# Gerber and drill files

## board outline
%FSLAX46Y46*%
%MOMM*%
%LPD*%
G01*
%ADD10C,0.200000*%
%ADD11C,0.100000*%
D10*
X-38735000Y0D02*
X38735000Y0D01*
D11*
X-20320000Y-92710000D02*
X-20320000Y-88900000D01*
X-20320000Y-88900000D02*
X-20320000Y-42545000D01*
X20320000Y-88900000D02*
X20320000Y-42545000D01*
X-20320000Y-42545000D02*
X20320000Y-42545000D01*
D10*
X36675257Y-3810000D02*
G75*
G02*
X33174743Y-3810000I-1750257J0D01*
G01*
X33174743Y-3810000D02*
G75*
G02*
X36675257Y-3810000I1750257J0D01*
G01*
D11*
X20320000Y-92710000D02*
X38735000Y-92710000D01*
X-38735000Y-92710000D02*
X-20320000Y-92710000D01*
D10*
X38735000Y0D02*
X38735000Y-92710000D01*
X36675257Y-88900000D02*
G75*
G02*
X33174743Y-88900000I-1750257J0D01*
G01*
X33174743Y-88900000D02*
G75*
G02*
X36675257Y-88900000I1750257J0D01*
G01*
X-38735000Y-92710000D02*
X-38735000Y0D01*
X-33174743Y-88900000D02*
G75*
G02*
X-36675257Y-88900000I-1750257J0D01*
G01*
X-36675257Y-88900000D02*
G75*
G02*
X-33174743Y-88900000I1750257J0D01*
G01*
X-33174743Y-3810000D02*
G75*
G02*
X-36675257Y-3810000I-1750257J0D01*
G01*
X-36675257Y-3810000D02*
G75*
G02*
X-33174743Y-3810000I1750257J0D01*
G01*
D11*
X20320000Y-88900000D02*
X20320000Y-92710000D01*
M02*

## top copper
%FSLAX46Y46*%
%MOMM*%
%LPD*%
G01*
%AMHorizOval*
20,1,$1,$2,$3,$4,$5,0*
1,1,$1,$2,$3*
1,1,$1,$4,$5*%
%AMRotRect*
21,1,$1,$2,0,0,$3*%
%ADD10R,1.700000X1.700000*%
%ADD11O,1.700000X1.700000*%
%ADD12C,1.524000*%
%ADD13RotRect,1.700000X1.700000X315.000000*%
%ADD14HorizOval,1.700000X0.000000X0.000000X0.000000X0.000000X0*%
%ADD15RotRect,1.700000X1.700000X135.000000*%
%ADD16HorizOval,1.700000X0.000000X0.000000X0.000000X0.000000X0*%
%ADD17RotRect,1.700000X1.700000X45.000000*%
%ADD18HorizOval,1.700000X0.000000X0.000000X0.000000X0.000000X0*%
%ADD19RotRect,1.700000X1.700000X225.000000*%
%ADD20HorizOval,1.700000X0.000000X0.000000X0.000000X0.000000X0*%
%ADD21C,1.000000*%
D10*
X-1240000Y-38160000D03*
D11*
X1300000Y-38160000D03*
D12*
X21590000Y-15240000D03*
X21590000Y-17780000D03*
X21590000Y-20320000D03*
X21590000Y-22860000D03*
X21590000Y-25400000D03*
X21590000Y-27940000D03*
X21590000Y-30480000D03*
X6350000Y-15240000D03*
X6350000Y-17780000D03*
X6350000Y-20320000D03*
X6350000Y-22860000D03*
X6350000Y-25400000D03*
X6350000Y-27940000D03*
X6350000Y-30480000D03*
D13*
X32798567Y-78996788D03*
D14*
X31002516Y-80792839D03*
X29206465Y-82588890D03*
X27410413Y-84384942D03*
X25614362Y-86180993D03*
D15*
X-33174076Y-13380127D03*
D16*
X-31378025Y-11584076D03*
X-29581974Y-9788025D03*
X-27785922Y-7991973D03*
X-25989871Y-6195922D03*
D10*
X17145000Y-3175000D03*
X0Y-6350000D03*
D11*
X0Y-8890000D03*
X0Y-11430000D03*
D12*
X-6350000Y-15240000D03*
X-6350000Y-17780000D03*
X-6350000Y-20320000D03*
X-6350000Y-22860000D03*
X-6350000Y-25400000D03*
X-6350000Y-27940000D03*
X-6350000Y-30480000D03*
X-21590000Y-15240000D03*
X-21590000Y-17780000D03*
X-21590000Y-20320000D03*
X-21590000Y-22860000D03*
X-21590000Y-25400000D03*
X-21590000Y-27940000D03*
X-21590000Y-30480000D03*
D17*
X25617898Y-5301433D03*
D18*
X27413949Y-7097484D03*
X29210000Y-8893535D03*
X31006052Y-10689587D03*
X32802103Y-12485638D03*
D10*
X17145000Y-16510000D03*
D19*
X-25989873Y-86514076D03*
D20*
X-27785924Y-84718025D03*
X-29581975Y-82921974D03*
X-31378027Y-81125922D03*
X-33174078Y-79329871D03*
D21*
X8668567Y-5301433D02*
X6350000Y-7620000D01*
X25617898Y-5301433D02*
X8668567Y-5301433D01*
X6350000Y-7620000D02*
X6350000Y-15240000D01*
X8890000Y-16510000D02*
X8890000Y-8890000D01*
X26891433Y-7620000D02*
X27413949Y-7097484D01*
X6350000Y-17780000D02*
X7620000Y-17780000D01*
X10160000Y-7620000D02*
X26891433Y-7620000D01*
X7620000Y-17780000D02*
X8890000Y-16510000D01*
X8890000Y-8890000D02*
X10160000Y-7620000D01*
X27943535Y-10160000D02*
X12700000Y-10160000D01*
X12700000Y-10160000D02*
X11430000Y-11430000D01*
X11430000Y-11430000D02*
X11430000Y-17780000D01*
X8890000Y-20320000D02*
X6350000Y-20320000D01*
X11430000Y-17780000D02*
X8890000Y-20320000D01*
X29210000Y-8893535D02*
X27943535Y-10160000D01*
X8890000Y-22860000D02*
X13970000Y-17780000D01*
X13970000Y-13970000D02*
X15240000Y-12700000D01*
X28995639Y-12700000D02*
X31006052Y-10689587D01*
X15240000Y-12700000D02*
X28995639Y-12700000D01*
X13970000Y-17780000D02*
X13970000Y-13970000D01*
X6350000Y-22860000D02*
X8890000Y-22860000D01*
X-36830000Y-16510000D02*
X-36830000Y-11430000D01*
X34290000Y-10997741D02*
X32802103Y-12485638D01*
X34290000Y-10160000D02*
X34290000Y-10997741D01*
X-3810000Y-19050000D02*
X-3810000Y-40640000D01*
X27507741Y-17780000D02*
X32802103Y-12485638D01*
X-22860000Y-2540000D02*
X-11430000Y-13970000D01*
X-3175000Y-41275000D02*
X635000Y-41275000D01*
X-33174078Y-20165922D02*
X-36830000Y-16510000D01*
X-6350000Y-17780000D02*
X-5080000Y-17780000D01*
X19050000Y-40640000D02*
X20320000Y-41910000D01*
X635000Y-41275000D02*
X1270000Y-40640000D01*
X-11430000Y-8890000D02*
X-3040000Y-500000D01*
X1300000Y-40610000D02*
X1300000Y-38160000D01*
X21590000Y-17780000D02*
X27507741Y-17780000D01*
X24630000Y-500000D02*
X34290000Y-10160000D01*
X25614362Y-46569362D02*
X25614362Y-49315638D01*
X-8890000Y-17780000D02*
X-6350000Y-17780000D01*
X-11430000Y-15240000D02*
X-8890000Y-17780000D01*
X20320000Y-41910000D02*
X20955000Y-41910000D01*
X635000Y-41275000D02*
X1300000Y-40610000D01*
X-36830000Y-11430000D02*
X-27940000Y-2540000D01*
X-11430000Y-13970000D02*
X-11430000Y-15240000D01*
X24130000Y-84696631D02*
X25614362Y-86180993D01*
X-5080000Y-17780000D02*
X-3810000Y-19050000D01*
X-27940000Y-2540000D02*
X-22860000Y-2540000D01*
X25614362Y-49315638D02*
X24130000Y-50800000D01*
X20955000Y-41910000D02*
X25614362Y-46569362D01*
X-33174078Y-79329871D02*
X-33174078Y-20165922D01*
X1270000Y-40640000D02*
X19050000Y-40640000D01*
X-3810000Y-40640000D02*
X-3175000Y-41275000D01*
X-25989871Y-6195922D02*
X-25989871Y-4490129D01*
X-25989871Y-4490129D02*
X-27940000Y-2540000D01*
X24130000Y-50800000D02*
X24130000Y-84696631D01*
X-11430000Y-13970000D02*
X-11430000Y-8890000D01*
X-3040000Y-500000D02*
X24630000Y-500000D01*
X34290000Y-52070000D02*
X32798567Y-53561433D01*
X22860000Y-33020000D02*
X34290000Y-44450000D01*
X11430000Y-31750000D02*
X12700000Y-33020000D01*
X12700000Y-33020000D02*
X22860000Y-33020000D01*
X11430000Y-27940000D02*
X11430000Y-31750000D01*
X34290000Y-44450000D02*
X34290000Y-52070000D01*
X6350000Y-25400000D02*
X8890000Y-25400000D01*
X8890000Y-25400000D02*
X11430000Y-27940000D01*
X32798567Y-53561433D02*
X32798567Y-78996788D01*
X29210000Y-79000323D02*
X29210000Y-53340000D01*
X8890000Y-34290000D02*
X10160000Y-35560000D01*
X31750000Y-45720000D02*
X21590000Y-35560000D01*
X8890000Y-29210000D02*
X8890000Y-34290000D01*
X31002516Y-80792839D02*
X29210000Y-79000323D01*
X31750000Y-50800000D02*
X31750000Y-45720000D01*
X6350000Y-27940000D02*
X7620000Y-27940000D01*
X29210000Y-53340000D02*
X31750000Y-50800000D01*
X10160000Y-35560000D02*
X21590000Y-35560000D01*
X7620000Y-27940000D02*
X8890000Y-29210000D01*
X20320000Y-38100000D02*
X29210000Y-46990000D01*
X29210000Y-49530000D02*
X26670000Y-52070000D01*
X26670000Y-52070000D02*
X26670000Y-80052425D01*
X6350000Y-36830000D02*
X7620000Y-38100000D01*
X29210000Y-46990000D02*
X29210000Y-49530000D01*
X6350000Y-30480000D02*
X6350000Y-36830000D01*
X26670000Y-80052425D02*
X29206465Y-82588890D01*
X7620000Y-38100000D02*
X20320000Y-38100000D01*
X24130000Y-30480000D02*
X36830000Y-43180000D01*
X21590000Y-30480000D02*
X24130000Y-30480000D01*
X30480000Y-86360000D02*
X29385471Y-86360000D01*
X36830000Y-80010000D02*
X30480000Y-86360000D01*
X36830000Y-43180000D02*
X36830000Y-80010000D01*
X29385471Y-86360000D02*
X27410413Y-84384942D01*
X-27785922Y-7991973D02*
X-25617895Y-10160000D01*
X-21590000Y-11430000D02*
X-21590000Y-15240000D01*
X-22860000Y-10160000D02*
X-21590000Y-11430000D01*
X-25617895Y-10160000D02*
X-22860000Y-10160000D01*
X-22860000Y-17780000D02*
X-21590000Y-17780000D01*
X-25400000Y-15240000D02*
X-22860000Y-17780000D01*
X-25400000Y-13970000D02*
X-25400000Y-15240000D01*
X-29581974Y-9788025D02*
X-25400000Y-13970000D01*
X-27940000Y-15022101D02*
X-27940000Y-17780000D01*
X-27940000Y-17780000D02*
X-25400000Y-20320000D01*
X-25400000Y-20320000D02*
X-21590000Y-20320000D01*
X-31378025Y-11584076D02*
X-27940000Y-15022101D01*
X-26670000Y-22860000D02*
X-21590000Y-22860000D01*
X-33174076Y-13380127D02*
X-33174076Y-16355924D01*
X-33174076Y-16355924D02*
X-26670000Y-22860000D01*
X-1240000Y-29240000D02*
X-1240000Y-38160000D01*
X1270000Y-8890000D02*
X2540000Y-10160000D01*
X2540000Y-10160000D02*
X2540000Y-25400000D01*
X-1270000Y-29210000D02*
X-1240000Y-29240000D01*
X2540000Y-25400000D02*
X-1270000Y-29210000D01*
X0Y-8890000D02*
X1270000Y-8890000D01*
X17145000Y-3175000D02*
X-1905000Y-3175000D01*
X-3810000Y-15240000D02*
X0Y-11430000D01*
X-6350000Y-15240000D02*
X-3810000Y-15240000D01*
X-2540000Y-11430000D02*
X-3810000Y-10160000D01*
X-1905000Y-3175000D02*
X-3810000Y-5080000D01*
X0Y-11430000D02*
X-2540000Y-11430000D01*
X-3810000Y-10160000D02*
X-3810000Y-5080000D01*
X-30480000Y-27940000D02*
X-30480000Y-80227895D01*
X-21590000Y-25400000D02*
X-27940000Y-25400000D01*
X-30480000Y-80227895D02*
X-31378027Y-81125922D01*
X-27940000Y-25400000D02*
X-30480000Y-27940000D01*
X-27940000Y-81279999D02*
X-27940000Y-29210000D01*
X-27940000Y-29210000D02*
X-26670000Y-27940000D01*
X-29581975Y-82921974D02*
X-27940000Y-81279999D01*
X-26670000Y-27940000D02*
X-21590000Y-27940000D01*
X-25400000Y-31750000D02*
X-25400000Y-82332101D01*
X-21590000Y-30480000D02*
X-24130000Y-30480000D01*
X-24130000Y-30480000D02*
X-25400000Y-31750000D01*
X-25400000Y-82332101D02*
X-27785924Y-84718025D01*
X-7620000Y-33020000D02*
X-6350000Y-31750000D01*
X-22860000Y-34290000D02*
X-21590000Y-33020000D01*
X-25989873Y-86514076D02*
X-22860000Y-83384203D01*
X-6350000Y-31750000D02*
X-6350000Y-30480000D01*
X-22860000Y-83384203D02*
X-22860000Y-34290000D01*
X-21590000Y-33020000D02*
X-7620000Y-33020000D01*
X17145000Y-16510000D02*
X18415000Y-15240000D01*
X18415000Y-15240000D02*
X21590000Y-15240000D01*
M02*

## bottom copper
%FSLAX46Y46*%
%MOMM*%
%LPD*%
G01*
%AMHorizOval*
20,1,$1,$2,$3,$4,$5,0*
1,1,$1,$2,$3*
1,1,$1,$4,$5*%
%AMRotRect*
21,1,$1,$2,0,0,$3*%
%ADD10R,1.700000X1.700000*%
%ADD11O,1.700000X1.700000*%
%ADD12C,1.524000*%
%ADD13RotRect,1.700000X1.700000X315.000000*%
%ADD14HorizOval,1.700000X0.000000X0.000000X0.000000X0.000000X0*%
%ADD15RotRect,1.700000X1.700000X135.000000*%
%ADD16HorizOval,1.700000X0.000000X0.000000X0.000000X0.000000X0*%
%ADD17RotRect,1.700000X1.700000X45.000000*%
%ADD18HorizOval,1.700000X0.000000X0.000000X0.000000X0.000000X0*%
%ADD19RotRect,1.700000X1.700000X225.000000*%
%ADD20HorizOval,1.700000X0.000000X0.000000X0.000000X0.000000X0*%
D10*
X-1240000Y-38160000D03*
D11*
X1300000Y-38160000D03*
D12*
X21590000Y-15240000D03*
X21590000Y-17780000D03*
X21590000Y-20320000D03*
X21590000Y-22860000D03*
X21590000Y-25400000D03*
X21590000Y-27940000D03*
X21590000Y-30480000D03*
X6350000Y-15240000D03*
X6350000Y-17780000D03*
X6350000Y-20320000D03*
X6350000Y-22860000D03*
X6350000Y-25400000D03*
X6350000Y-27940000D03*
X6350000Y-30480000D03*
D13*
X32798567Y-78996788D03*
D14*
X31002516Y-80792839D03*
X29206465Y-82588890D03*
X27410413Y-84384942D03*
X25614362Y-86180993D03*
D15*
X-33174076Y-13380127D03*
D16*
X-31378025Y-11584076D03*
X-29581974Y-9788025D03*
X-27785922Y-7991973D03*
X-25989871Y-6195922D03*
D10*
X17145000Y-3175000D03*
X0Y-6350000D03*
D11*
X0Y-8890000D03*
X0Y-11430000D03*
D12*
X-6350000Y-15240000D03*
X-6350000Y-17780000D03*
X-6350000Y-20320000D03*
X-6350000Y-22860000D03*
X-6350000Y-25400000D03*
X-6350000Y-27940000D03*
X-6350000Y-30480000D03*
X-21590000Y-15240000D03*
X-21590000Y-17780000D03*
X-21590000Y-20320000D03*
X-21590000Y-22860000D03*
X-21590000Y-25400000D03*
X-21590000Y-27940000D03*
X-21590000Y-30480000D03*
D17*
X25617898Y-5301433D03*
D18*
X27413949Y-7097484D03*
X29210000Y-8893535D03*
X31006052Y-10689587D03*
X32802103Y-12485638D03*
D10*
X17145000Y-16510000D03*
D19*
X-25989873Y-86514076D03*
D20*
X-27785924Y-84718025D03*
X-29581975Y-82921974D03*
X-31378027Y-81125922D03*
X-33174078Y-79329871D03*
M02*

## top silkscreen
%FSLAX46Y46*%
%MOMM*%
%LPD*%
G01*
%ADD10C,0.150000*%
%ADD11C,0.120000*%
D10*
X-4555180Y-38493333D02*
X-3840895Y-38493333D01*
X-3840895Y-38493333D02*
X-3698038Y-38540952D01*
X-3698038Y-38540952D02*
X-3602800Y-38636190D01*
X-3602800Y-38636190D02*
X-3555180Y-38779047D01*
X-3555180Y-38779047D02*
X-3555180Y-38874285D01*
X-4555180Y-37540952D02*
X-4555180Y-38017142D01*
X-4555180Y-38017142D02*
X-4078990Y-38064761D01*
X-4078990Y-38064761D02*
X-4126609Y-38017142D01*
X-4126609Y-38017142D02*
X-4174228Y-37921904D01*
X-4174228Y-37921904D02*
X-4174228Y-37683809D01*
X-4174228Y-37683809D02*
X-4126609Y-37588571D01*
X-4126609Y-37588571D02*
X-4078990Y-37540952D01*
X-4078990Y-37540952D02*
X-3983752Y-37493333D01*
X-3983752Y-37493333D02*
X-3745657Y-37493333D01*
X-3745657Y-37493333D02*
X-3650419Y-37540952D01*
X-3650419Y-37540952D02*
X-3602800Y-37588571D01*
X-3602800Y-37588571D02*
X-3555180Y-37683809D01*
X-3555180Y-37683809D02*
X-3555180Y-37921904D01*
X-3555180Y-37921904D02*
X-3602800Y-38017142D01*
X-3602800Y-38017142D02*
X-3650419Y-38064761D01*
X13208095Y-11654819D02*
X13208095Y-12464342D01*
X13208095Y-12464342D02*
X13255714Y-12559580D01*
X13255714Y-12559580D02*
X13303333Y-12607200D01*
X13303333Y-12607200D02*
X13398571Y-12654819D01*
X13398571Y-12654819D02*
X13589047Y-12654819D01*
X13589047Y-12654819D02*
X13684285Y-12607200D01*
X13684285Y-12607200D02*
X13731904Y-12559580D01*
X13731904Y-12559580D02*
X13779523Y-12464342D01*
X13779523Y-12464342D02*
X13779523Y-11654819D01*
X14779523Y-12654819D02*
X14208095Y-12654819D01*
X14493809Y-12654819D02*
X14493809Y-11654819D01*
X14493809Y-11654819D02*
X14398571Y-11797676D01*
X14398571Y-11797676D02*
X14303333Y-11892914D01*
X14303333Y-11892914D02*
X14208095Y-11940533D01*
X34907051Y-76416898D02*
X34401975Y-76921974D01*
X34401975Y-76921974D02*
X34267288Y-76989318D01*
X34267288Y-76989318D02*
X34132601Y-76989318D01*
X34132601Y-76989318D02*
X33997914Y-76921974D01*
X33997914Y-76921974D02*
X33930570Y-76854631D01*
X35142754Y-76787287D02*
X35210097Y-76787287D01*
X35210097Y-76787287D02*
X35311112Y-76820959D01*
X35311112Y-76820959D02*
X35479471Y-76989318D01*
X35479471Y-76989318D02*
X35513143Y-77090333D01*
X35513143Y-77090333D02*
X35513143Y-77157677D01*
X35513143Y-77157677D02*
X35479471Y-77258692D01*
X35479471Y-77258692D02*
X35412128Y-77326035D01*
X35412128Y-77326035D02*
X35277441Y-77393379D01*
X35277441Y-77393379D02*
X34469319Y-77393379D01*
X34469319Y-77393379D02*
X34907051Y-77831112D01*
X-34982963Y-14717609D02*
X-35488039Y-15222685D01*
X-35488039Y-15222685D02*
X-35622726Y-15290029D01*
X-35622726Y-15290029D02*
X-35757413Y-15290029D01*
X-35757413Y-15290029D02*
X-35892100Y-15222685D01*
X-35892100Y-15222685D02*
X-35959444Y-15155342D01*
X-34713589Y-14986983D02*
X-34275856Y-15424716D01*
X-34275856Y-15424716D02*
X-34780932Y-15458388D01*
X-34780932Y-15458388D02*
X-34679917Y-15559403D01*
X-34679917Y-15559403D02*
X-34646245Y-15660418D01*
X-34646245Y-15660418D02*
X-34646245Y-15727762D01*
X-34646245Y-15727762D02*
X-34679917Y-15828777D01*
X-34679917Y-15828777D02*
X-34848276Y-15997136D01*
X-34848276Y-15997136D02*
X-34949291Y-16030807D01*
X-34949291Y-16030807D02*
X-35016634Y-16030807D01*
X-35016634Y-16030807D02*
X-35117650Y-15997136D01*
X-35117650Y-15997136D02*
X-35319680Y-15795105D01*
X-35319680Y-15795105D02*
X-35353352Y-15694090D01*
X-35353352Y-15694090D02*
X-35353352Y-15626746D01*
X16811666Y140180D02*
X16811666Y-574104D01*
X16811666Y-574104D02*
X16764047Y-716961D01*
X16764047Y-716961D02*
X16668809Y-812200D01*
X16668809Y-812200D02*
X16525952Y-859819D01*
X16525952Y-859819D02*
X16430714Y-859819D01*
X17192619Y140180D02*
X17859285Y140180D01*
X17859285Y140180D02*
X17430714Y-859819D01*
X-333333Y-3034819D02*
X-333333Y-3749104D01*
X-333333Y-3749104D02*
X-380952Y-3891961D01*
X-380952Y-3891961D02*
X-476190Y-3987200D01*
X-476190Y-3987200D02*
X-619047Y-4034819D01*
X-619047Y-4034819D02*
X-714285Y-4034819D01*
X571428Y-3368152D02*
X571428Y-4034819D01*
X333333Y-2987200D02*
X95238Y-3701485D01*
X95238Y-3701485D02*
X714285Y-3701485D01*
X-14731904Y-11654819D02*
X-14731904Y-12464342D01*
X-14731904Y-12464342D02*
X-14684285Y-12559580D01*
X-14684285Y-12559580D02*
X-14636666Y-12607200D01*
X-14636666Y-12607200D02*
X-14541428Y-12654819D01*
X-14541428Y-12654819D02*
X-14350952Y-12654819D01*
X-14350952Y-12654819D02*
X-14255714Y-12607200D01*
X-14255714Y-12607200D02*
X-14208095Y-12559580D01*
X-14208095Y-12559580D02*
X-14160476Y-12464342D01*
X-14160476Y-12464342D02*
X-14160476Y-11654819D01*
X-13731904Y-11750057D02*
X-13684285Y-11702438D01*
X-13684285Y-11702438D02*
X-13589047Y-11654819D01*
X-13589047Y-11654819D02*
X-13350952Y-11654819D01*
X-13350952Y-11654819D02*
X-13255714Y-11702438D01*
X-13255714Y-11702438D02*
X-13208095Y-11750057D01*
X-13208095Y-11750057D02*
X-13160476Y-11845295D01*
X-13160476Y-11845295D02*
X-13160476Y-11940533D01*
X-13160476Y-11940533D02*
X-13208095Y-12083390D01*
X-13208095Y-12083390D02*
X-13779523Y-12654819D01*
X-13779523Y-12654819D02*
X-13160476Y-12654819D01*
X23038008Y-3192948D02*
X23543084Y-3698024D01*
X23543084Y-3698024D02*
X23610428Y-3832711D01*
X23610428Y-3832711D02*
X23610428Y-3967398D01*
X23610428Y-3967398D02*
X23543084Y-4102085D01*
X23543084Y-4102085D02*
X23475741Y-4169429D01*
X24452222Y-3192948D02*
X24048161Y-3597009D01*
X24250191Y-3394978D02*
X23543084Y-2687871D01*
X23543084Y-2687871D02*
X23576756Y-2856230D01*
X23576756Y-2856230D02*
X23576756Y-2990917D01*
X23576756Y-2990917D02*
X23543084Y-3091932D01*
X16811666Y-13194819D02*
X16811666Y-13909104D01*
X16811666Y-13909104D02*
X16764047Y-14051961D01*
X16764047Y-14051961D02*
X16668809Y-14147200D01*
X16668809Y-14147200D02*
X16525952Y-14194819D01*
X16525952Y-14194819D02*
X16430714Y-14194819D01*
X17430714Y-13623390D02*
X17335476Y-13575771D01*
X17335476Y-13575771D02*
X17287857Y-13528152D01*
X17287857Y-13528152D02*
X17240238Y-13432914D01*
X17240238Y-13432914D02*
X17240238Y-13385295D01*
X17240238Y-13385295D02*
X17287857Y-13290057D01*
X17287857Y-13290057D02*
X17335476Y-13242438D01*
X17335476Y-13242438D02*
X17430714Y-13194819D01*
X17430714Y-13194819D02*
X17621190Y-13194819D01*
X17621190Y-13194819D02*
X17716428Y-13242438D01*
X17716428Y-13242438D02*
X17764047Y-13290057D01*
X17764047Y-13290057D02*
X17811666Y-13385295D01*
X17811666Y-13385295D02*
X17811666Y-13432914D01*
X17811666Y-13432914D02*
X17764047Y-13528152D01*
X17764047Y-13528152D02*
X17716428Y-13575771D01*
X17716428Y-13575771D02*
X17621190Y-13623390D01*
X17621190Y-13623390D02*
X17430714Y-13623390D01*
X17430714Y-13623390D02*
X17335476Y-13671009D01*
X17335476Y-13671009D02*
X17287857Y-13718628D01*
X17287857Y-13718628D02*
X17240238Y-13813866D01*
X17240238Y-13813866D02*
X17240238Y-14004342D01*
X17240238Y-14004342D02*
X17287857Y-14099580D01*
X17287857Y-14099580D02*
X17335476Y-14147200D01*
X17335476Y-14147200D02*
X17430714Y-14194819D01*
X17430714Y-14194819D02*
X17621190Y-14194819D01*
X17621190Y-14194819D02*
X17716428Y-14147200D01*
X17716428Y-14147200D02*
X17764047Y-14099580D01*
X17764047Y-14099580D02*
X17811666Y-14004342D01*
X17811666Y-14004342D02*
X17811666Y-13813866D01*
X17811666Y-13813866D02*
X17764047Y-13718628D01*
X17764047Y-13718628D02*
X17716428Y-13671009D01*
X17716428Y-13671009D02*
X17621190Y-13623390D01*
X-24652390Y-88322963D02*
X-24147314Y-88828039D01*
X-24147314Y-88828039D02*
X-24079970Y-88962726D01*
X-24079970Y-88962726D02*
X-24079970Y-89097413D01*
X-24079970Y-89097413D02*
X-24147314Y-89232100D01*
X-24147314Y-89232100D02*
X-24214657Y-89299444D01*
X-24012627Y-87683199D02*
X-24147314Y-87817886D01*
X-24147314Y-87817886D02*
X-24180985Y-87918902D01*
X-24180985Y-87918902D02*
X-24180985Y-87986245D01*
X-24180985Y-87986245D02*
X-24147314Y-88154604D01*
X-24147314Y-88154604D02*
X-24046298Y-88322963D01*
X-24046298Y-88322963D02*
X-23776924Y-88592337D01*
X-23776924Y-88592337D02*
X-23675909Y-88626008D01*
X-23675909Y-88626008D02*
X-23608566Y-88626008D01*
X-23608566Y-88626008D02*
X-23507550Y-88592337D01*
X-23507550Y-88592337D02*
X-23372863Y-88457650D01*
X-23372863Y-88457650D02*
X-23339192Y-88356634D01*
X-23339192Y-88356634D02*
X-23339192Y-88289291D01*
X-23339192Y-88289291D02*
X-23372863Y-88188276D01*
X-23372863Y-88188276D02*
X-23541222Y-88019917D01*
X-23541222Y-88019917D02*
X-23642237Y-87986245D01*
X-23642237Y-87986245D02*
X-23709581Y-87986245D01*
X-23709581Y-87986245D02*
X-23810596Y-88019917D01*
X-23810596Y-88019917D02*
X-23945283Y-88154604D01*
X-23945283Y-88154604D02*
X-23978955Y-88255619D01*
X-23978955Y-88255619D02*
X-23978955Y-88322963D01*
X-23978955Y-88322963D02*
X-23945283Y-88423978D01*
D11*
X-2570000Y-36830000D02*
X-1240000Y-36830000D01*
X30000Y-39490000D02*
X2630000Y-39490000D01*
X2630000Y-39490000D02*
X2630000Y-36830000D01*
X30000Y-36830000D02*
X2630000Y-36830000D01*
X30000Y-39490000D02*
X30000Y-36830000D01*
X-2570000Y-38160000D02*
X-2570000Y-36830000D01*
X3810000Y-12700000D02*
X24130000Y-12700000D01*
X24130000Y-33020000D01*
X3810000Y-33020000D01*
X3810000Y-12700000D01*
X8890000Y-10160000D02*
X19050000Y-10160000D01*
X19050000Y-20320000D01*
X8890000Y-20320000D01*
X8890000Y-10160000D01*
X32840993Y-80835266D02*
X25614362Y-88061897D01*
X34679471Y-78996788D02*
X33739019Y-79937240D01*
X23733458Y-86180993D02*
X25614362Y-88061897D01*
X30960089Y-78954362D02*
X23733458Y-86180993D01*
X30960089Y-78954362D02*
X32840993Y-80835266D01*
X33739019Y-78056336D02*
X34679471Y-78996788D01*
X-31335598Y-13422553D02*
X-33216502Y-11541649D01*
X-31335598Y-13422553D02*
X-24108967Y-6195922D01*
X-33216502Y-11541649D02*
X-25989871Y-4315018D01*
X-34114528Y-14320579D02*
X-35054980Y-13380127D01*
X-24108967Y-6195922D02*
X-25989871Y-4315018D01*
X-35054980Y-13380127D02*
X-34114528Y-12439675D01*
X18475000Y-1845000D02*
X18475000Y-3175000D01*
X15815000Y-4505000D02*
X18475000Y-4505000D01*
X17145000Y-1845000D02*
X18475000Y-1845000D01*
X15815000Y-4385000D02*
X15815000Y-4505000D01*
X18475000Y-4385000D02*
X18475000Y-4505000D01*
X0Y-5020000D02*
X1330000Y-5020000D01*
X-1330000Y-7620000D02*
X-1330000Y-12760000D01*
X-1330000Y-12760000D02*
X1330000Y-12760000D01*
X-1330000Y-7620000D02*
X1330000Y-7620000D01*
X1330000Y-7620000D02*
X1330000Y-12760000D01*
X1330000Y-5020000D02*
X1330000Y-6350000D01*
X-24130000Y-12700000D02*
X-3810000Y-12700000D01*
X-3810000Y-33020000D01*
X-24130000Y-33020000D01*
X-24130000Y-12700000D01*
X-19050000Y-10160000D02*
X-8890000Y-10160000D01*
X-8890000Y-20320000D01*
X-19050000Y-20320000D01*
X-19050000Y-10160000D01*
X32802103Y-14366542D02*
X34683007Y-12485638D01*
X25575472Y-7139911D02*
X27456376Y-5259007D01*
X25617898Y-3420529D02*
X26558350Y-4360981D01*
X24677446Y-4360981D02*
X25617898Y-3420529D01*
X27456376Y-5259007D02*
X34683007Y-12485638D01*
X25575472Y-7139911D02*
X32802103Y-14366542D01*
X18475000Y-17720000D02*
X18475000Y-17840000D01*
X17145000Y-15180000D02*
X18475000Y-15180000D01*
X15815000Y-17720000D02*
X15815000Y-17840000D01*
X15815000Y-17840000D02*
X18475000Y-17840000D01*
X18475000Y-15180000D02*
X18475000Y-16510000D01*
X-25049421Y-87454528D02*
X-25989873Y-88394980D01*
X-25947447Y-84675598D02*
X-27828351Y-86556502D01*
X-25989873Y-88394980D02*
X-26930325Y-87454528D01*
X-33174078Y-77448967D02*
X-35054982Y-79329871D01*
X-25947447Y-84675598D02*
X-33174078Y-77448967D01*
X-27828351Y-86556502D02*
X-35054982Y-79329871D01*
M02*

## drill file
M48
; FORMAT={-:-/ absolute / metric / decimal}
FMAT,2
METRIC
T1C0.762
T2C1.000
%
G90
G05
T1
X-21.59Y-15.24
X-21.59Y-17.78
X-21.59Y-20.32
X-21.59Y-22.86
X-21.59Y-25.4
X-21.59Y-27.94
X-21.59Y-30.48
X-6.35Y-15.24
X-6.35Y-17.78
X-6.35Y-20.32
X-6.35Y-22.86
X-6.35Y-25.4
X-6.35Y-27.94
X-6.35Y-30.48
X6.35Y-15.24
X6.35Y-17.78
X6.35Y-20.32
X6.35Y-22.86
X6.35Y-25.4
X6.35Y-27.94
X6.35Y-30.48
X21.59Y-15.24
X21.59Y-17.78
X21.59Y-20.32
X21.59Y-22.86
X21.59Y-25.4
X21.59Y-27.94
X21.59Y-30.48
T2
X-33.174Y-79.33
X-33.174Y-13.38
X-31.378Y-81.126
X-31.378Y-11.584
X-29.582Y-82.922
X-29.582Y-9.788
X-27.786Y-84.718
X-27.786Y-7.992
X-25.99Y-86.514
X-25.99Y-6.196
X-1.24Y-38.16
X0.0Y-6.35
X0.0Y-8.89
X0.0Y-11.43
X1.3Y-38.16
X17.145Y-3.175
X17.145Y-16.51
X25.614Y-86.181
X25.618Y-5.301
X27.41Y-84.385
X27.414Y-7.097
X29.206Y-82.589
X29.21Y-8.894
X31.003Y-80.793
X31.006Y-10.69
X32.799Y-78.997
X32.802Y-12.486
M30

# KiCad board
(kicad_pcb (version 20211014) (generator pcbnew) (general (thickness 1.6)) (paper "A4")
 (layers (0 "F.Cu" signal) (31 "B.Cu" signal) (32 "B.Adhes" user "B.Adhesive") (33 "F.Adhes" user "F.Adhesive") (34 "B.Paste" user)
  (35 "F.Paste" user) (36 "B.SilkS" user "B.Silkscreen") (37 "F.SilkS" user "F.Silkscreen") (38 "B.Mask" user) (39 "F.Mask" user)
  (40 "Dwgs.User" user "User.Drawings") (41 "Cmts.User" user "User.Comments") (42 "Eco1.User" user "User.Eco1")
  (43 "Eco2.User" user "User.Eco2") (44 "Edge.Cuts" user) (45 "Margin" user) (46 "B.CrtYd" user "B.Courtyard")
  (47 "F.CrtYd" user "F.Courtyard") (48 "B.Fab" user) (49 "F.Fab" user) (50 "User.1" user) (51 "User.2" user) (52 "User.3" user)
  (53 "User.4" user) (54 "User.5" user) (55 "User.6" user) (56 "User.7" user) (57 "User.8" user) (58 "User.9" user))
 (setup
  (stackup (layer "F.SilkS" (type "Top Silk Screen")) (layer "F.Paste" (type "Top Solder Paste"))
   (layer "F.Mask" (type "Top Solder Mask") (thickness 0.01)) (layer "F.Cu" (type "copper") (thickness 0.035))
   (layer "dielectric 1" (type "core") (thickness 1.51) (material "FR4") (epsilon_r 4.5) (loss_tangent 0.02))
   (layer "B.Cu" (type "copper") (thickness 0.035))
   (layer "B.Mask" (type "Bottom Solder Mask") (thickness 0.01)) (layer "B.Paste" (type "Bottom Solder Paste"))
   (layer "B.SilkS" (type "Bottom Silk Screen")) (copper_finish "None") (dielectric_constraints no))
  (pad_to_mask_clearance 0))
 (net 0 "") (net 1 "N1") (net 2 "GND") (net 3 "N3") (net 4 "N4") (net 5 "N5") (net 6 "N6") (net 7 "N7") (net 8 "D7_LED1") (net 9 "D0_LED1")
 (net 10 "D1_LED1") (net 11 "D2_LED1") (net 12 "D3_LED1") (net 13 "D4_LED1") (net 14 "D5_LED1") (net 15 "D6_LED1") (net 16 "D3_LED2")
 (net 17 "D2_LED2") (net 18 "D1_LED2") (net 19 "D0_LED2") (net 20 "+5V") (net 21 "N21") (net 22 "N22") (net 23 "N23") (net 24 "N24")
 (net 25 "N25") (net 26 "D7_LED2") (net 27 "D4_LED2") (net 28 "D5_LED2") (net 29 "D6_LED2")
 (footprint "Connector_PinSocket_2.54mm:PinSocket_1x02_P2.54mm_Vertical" (layer "F.Cu") (at -1.24 38.16 90)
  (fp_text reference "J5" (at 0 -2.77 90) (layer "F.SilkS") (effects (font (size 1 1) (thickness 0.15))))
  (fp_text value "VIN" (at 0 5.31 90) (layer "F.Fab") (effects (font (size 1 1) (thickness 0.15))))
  (fp_line (start 1.33 -1.33) (end 1.33 0) (layer "F.SilkS") (width 0.12))
  (fp_line (start -1.33 1.27) (end -1.33 3.87) (layer "F.SilkS") (width 0.12))
  (fp_line (start -1.33 3.87) (end 1.33 3.87) (layer "F.SilkS") (width 0.12))
  (fp_line (start 1.33 1.27) (end 1.33 3.87) (layer "F.SilkS") (width 0.12))
  (fp_line (start -1.33 1.27) (end 1.33 1.27) (layer "F.SilkS") (width 0.12))
  (fp_line (start 0 -1.33) (end 1.33 -1.33) (layer "F.SilkS") (width 0.12))
  (pad "1" thru_hole rect (at 0 0 90) (size 1.7 1.7) (drill 1) (layers *.Cu *.Mask) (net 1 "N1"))
  (pad "2" thru_hole oval (at 0 2.54 90) (size 1.7 1.7) (drill 1) (layers *.Cu *.Mask) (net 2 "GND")))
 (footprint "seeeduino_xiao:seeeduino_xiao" (layer "F.Cu") (at 13.97 12.7)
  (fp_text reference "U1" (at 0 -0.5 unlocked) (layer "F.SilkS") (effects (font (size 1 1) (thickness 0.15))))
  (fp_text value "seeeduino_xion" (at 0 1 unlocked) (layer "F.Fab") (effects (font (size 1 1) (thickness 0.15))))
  (fp_rect (start -10.16 0) (end 10.16 20.32) (layer "F.SilkS") (width 0.12) (fill none))
  (fp_rect (start -5.08 -2.54) (end 5.08 7.62) (layer "F.SilkS") (width 0.12) (fill none))
  (pad "1" thru_hole circle (at 7.62 2.54) (size 1.524 1.524) (drill 0.762) (layers *.Cu *.Mask) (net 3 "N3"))
  (pad "2" thru_hole circle (at 7.62 5.08) (size 1.524 1.524) (drill 0.762) (layers *.Cu *.Mask) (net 2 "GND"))
  (pad "3" thru_hole circle (at 7.62 7.62) (size 1.524 1.524) (drill 0.762) (layers *.Cu *.Mask) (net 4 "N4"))
  (pad "4" thru_hole circle (at 7.62 10.16) (size 1.524 1.524) (drill 0.762) (layers *.Cu *.Mask) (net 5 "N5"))
  (pad "5" thru_hole circle (at 7.62 12.7) (size 1.524 1.524) (drill 0.762) (layers *.Cu *.Mask) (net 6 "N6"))
  (pad "6" thru_hole circle (at 7.62 15.24) (size 1.524 1.524) (drill 0.762) (layers *.Cu *.Mask) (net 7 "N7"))
  (pad "7" thru_hole circle (at 7.62 17.78) (size 1.524 1.524) (drill 0.762) (layers *.Cu *.Mask) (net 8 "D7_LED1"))
  (pad "8" thru_hole circle (at -7.62 2.54) (size 1.524 1.524) (drill 0.762) (layers *.Cu *.Mask) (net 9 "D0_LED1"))
  (pad "9" thru_hole circle (at -7.62 5.08) (size 1.524 1.524) (drill 0.762) (layers *.Cu *.Mask) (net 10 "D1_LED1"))
  (pad "10" thru_hole circle (at -7.62 7.62) (size 1.524 1.524) (drill 0.762) (layers *.Cu *.Mask) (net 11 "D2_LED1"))
  (pad "11" thru_hole circle (at -7.62 10.16) (size 1.524 1.524) (drill 0.762) (layers *.Cu *.Mask) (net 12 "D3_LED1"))
  (pad "12" thru_hole circle (at -7.62 12.7) (size 1.524 1.524) (drill 0.762) (layers *.Cu *.Mask) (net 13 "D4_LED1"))
  (pad "13" thru_hole circle (at -7.62 15.24) (size 1.524 1.524) (drill 0.762) (layers *.Cu *.Mask) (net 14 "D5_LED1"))
  (pad "14" thru_hole circle (at -7.62 17.78) (size 1.524 1.524) (drill 0.762) (layers *.Cu *.Mask) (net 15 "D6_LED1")))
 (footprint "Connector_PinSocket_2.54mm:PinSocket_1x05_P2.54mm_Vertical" (layer "F.Cu") (at 32.798567 78.996788 -45)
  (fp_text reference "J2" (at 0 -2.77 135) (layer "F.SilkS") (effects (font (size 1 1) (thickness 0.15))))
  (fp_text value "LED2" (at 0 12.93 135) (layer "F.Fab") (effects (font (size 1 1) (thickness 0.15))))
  (fp_line (start 1.33 1.27) (end 1.33 11.49) (layer "F.SilkS") (width 0.12))
  (fp_line (start 1.33 -1.33) (end 1.33 0) (layer "F.SilkS") (width 0.12))
  (fp_line (start -1.33 11.49) (end 1.33 11.49) (layer "F.SilkS") (width 0.12))
  (fp_line (start -1.33 1.27) (end -1.33 11.49) (layer "F.SilkS") (width 0.12))
  (fp_line (start -1.33 1.27) (end 1.33 1.27) (layer "F.SilkS") (width 0.12))
  (fp_line (start 0 -1.33) (end 1.33 -1.33) (layer "F.SilkS") (width 0.12))
  (pad "1" thru_hole rect (at 0 0 315) (size 1.7 1.7) (drill 1) (layers *.Cu *.Mask) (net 13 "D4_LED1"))
  (pad "2" thru_hole oval (at 0 2.54 315) (size 1.7 1.7) (drill 1) (layers *.Cu *.Mask) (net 14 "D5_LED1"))
  (pad "3" thru_hole oval (at 0 5.08 315) (size 1.7 1.7) (drill 1) (layers *.Cu *.Mask) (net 15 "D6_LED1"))
  (pad "4" thru_hole oval (at 0 7.62 315) (size 1.7 1.7) (drill 1) (layers *.Cu *.Mask) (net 8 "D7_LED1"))
  (pad "5" thru_hole oval (at 0 10.16 315) (size 1.7 1.7) (drill 1) (layers *.Cu *.Mask) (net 2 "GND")))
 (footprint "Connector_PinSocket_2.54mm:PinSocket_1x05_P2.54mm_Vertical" (layer "F.Cu") (at -33.174076 13.380127 135)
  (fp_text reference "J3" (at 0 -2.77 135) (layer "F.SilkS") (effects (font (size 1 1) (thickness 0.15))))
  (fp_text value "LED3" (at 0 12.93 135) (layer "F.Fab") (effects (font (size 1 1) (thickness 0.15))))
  (fp_line (start -1.33 1.27) (end 1.33 1.27) (layer "F.SilkS") (width 0.12))
  (fp_line (start -1.33 1.27) (end -1.33 11.49) (layer "F.SilkS") (width 0.12))
  (fp_line (start 1.33 1.27) (end 1.33 11.49) (layer "F.SilkS") (width 0.12))
  (fp_line (start 0 -1.33) (end 1.33 -1.33) (layer "F.SilkS") (width 0.12))
  (fp_line (start -1.33 11.49) (end 1.33 11.49) (layer "F.SilkS") (width 0.12))
  (fp_line (start 1.33 -1.33) (end 1.33 0) (layer "F.SilkS") (width 0.12))
  (pad "1" thru_hole rect (at 0 0 135) (size 1.7 1.7) (drill 1) (layers *.Cu *.Mask) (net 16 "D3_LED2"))
  (pad "2" thru_hole oval (at 0 2.54 135) (size 1.7 1.7) (drill 1) (layers *.Cu *.Mask) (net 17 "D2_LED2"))
  (pad "3" thru_hole oval (at 0 5.08 135) (size 1.7 1.7) (drill 1) (layers *.Cu *.Mask) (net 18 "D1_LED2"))
  (pad "4" thru_hole oval (at 0 7.62 135) (size 1.7 1.7) (drill 1) (layers *.Cu *.Mask) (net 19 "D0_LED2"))
  (pad "5" thru_hole oval (at 0 10.16 135) (size 1.7 1.7) (drill 1) (layers *.Cu *.Mask) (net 2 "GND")))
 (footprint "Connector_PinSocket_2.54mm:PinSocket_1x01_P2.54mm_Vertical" (layer "F.Cu") (at 17.145 3.175)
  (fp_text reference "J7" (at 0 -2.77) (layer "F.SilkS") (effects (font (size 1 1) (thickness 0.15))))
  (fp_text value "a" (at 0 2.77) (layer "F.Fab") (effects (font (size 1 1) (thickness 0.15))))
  (fp_line (start 1.33 -1.33) (end 1.33 0) (layer "F.SilkS") (width 0.12))
  (fp_line (start -1.33 1.33) (end 1.33 1.33) (layer "F.SilkS") (width 0.12))
  (fp_line (start 0 -1.33) (end 1.33 -1.33) (layer "F.SilkS") (width 0.12))
  (fp_line (start -1.33 1.21) (end -1.33 1.33) (layer "F.SilkS") (width 0.12))
  (fp_line (start 1.33 1.21) (end 1.33 1.33) (layer "F.SilkS") (width 0.12))
  (pad "1" thru_hole rect (at 0 0) (size 1.7 1.7) (drill 1) (layers *.Cu *.Mask) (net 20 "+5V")))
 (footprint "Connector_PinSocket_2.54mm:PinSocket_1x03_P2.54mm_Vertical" (layer "F.Cu") (at 0 6.35)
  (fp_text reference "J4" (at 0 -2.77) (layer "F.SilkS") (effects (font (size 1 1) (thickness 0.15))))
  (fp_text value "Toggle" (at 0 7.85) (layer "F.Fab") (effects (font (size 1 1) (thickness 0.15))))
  (fp_line (start 0 -1.33) (end 1.33 -1.33) (layer "F.SilkS") (width 0.12))
  (fp_line (start -1.33 1.27) (end -1.33 6.41) (layer "F.SilkS") (width 0.12))
  (fp_line (start -1.33 6.41) (end 1.33 6.41) (layer "F.SilkS") (width 0.12))
  (fp_line (start -1.33 1.27) (end 1.33 1.27) (layer "F.SilkS") (width 0.12))
  (fp_line (start 1.33 1.27) (end 1.33 6.41) (layer "F.SilkS") (width 0.12))
  (fp_line (start 1.33 -1.33) (end 1.33 0) (layer "F.SilkS") (width 0.12))
  (pad "1" thru_hole rect (at 0 0) (size 1.7 1.7) (drill 1) (layers *.Cu *.Mask) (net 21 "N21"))
  (pad "2" thru_hole oval (at 0 2.54) (size 1.7 1.7) (drill 1) (layers *.Cu *.Mask) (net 1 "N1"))
  (pad "3" thru_hole oval (at 0 5.08) (size 1.7 1.7) (drill 1) (layers *.Cu *.Mask) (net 20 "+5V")))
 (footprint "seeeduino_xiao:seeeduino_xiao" (layer "F.Cu") (at -13.97 12.7)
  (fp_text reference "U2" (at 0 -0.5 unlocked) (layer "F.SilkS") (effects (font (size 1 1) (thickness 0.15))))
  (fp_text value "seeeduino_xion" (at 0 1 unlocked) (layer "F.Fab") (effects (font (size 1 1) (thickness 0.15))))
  (fp_rect (start -10.16 0) (end 10.16 20.32) (layer "F.SilkS") (width 0.12) (fill none))
  (fp_rect (start -5.08 -2.54) (end 5.08 7.62) (layer "F.SilkS") (width 0.12) (fill none))
  (pad "1" thru_hole circle (at 7.62 2.54) (size 1.524 1.524) (drill 0.762) (layers *.Cu *.Mask) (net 20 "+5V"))
  (pad "2" thru_hole circle (at 7.62 5.08) (size 1.524 1.524) (drill 0.762) (layers *.Cu *.Mask) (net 2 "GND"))
  (pad "3" thru_hole circle (at 7.62 7.62) (size 1.524 1.524) (drill 0.762) (layers *.Cu *.Mask) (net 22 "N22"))
  (pad "4" thru_hole circle (at 7.62 10.16) (size 1.524 1.524) (drill 0.762) (layers *.Cu *.Mask) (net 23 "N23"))
  (pad "5" thru_hole circle (at 7.62 12.7) (size 1.524 1.524) (drill 0.762) (layers *.Cu *.Mask) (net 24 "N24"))
  (pad "6" thru_hole circle (at 7.62 15.24) (size 1.524 1.524) (drill 0.762) (layers *.Cu *.Mask) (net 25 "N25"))
  (pad "7" thru_hole circle (at 7.62 17.78) (size 1.524 1.524) (drill 0.762) (layers *.Cu *.Mask) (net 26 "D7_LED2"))
  (pad "8" thru_hole circle (at -7.62 2.54) (size 1.524 1.524) (drill 0.762) (layers *.Cu *.Mask) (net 19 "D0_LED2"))
  (pad "9" thru_hole circle (at -7.62 5.08) (size 1.524 1.524) (drill 0.762) (layers *.Cu *.Mask) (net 18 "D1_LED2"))
  (pad "10" thru_hole circle (at -7.62 7.62) (size 1.524 1.524) (drill 0.762) (layers *.Cu *.Mask) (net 17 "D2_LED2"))
  (pad "11" thru_hole circle (at -7.62 10.16) (size 1.524 1.524) (drill 0.762) (layers *.Cu *.Mask) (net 16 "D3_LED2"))
  (pad "12" thru_hole circle (at -7.62 12.7) (size 1.524 1.524) (drill 0.762) (layers *.Cu *.Mask) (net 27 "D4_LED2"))
  (pad "13" thru_hole circle (at -7.62 15.24) (size 1.524 1.524) (drill 0.762) (layers *.Cu *.Mask) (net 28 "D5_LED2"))
  (pad "14" thru_hole circle (at -7.62 17.78) (size 1.524 1.524) (drill 0.762) (layers *.Cu *.Mask) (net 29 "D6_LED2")))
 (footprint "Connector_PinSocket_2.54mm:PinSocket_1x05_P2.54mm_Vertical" (layer "F.Cu") (at 25.617898 5.301433 45)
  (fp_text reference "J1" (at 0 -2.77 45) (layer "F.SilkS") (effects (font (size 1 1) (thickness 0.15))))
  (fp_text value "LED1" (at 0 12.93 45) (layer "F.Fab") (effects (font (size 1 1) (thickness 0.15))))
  (fp_line (start -1.33 11.49) (end 1.33 11.49) (layer "F.SilkS") (width 0.12))
  (fp_line (start -1.33 1.27) (end 1.33 1.27) (layer "F.SilkS") (width 0.12))
  (fp_line (start 1.33 -1.33) (end 1.33 0) (layer "F.SilkS") (width 0.12))
  (fp_line (start 0 -1.33) (end 1.33 -1.33) (layer "F.SilkS") (width 0.12))
  (fp_line (start 1.33 1.27) (end 1.33 11.49) (layer "F.SilkS") (width 0.12))
  (fp_line (start -1.33 1.27) (end -1.33 11.49) (layer "F.SilkS") (width 0.12))
  (pad "1" thru_hole rect (at 0 0 45) (size 1.7 1.7) (drill 1) (layers *.Cu *.Mask) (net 9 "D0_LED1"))
  (pad "2" thru_hole oval (at 0 2.54 45) (size 1.7 1.7) (drill 1) (layers *.Cu *.Mask) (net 10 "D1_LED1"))
  (pad "3" thru_hole oval (at 0 5.08 45) (size 1.7 1.7) (drill 1) (layers *.Cu *.Mask) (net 11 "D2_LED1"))
  (pad "4" thru_hole oval (at 0 7.62 45) (size 1.7 1.7) (drill 1) (layers *.Cu *.Mask) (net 12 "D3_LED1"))
  (pad "5" thru_hole oval (at 0 10.16 45) (size 1.7 1.7) (drill 1) (layers *.Cu *.Mask) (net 2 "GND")))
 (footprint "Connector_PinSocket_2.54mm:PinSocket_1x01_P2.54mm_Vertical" (layer "F.Cu") (at 17.145 16.51)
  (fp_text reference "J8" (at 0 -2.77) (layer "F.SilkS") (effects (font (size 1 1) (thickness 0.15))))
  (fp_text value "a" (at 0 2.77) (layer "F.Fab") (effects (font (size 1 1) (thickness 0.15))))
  (fp_line (start 1.33 1.21) (end 1.33 1.33) (layer "F.SilkS") (width 0.12))
  (fp_line (start 0 -1.33) (end 1.33 -1.33) (layer "F.SilkS") (width 0.12))
  (fp_line (start -1.33 1.21) (end -1.33 1.33) (layer "F.SilkS") (width 0.12))
  (fp_line (start -1.33 1.33) (end 1.33 1.33) (layer "F.SilkS") (width 0.12))
  (fp_line (start 1.33 -1.33) (end 1.33 0) (layer "F.SilkS") (width 0.12))
  (pad "1" thru_hole rect (at 0 0) (size 1.7 1.7) (drill 1) (layers *.Cu *.Mask) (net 3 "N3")))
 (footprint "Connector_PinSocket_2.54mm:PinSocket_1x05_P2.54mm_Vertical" (layer "F.Cu") (at -25.989873 86.514076 -135)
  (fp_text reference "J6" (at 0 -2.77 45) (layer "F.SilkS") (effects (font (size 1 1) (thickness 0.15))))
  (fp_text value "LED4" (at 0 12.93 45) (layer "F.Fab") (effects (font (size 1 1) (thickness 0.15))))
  (fp_line (start 0 -1.33) (end 1.33 -1.33) (layer "F.SilkS") (width 0.12))
  (fp_line (start -1.33 1.27) (end 1.33 1.27) (layer "F.SilkS") (width 0.12))
  (fp_line (start 1.33 -1.33) (end 1.33 0) (layer "F.SilkS") (width 0.12))
  (fp_line (start -1.33 11.49) (end 1.33 11.49) (layer "F.SilkS") (width 0.12))
  (fp_line (start -1.33 1.27) (end -1.33 11.49) (layer "F.SilkS") (width 0.12))
  (fp_line (start 1.33 1.27) (end 1.33 11.49) (layer "F.SilkS") (width 0.12))
  (pad "1" thru_hole rect (at 0 0 225) (size 1.7 1.7) (drill 1) (layers *.Cu *.Mask) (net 26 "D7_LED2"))
  (pad "2" thru_hole oval (at 0 2.54 225) (size 1.7 1.7) (drill 1) (layers *.Cu *.Mask) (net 29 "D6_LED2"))
  (pad "3" thru_hole oval (at 0 5.08 225) (size 1.7 1.7) (drill 1) (layers *.Cu *.Mask) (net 28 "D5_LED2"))
  (pad "4" thru_hole oval (at 0 7.62 225) (size 1.7 1.7) (drill 1) (layers *.Cu *.Mask) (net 27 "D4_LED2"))
  (pad "5" thru_hole oval (at 0 10.16 225) (size 1.7 1.7) (drill 1) (layers *.Cu *.Mask) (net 2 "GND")))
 (gr_line (start -38.735 0) (end 38.735 0) (layer "Edge.Cuts") (width 0.2))
 (gr_line (start -20.32 92.71) (end -20.32 88.9) (layer "Edge.Cuts") (width 0.1))
 (gr_line (start -20.32 88.9) (end -20.32 42.545) (layer "Edge.Cuts") (width 0.1))
 (gr_line (start 20.32 88.9) (end 20.32 42.545) (layer "Edge.Cuts") (width 0.1))
 (gr_line (start -20.32 42.545) (end 20.32 42.545) (layer "Edge.Cuts") (width 0.1))
 (gr_circle (center 34.925 3.81) (end 36.675257 3.81) (layer "Edge.Cuts") (width 0.2) (fill none))
 (gr_line (start 20.32 92.71) (end 38.735 92.71) (layer "Edge.Cuts") (width 0.1))
 (gr_line (start -38.735 92.71) (end -20.32 92.71) (layer "Edge.Cuts") (width 0.1))
 (gr_line (start 38.735 0) (end 38.735 92.71) (layer "Edge.Cuts") (width 0.2))
 (gr_circle (center 34.925 88.9) (end 36.675257 88.9) (layer "Edge.Cuts") (width 0.2) (fill none))
 (gr_line (start -38.735 92.71) (end -38.735 0) (layer "Edge.Cuts") (width 0.2))
 (gr_circle (center -34.925 88.9) (end -33.174743 88.9) (layer "Edge.Cuts") (width 0.2) (fill none))
 (gr_circle (center -34.925 3.81) (end -33.174743 3.81) (layer "Edge.Cuts") (width 0.2) (fill none))
 (gr_line (start 20.32 88.9) (end 20.32 92.71) (layer "Edge.Cuts") (width 0.1))
 (segment (start 8.668567 5.301433) (end 6.35 7.62) (width 1) (layer "F.Cu") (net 9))
 (segment (start 25.617898 5.301433) (end 8.668567 5.301433) (width 1) (layer "F.Cu") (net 9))
 (segment (start 6.35 7.62) (end 6.35 15.24) (width 1) (layer "F.Cu") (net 9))
 (segment (start 8.89 16.51) (end 8.89 8.89) (width 1) (layer "F.Cu") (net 10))
 (segment (start 26.891433 7.62) (end 27.413949 7.097484) (width 1) (layer "F.Cu") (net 10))
 (segment (start 6.35 17.78) (end 7.62 17.78) (width 1) (layer "F.Cu") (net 10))
 (segment (start 10.16 7.62) (end 26.891433 7.62) (width 1) (layer "F.Cu") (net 10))
 (segment (start 7.62 17.78) (end 8.89 16.51) (width 1) (layer "F.Cu") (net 10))
 (segment (start 8.89 8.89) (end 10.16 7.62) (width 1) (layer "F.Cu") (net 10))
 (segment (start 27.943535 10.16) (end 12.7 10.16) (width 1) (layer "F.Cu") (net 11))
 (segment (start 12.7 10.16) (end 11.43 11.43) (width 1) (layer "F.Cu") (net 11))
 (segment (start 11.43 11.43) (end 11.43 17.78) (width 1) (layer "F.Cu") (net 11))
 (segment (start 8.89 20.32) (end 6.35 20.32) (width 1) (layer "F.Cu") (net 11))
 (segment (start 11.43 17.78) (end 8.89 20.32) (width 1) (layer "F.Cu") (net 11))
 (segment (start 29.21 8.893535) (end 27.943535 10.16) (width 1) (layer "F.Cu") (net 11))
 (segment (start 8.89 22.86) (end 13.97 17.78) (width 1) (layer "F.Cu") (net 12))
 (segment (start 13.97 13.97) (end 15.24 12.7) (width 1) (layer "F.Cu") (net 12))
 (segment (start 28.995639 12.7) (end 31.006052 10.689587) (width 1) (layer "F.Cu") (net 12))
 (segment (start 15.24 12.7) (end 28.995639 12.7) (width 1) (layer "F.Cu") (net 12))
 (segment (start 13.97 17.78) (end 13.97 13.97) (width 1) (layer "F.Cu") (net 12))
 (segment (start 6.35 22.86) (end 8.89 22.86) (width 1) (layer "F.Cu") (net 12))
 (segment (start -36.83 16.51) (end -36.83 11.43) (width 1) (layer "F.Cu") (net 2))
 (segment (start 34.29 10.997741) (end 32.802103 12.485638) (width 1) (layer "F.Cu") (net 2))
 (segment (start 34.29 10.16) (end 34.29 10.997741) (width 1) (layer "F.Cu") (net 2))
 (segment (start -3.81 19.05) (end -3.81 40.64) (width 1) (layer "F.Cu") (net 2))
 (segment (start 27.507741 17.78) (end 32.802103 12.485638) (width 1) (layer "F.Cu") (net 2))
 (segment (start -22.86 2.54) (end -11.43 13.97) (width 1) (layer "F.Cu") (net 2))
 (segment (start -3.175 41.275) (end 0.635 41.275) (width 1) (layer "F.Cu") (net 2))
 (segment (start -33.174078 20.165922) (end -36.83 16.51) (width 1) (layer "F.Cu") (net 2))
 (segment (start -6.35 17.78) (end -5.08 17.78) (width 1) (layer "F.Cu") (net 2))
 (segment (start 19.05 40.64) (end 20.32 41.91) (width 1) (layer "F.Cu") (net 2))
 (segment (start 0.635 41.275) (end 1.27 40.64) (width 1) (layer "F.Cu") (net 2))
 (segment (start -11.43 8.89) (end -3.04 0.5) (width 1) (layer "F.Cu") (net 2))
 (segment (start 1.3 40.61) (end 1.3 38.16) (width 1) (layer "F.Cu") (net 2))
 (segment (start 21.59 17.78) (end 27.507741 17.78) (width 1) (layer "F.Cu") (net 2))
 (segment (start 24.63 0.5) (end 34.29 10.16) (width 1) (layer "F.Cu") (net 2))
 (segment (start 25.614362 46.569362) (end 25.614362 49.315638) (width 1) (layer "F.Cu") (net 2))
 (segment (start -8.89 17.78) (end -6.35 17.78) (width 1) (layer "F.Cu") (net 2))
 (segment (start -11.43 15.24) (end -8.89 17.78) (width 1) (layer "F.Cu") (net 2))
 (segment (start 20.32 41.91) (end 20.955 41.91) (width 1) (layer "F.Cu") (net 2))
 (segment (start 0.635 41.275) (end 1.3 40.61) (width 1) (layer "F.Cu") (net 2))
 (segment (start -36.83 11.43) (end -27.94 2.54) (width 1) (layer "F.Cu") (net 2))
 (segment (start -11.43 13.97) (end -11.43 15.24) (width 1) (layer "F.Cu") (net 2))
 (segment (start 24.13 84.696631) (end 25.614362 86.180993) (width 1) (layer "F.Cu") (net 2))
 (segment (start -5.08 17.78) (end -3.81 19.05) (width 1) (layer "F.Cu") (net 2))
 (segment (start -27.94 2.54) (end -22.86 2.54) (width 1) (layer "F.Cu") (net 2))
 (segment (start 25.614362 49.315638) (end 24.13 50.8) (width 1) (layer "F.Cu") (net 2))
 (segment (start 20.955 41.91) (end 25.614362 46.569362) (width 1) (layer "F.Cu") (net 2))
 (segment (start -33.174078 79.329871) (end -33.174078 20.165922) (width 1) (layer "F.Cu") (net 2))
 (segment (start 1.27 40.64) (end 19.05 40.64) (width 1) (layer "F.Cu") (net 2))
 (segment (start -3.81 40.64) (end -3.175 41.275) (width 1) (layer "F.Cu") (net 2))
 (segment (start -25.989871 6.195922) (end -25.989871 4.490129) (width 1) (layer "F.Cu") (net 2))
 (segment (start -25.989871 4.490129) (end -27.94 2.54) (width 1) (layer "F.Cu") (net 2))
 (segment (start 24.13 50.8) (end 24.13 84.696631) (width 1) (layer "F.Cu") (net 2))
 (segment (start -11.43 13.97) (end -11.43 8.89) (width 1) (layer "F.Cu") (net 2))
 (segment (start -3.04 0.5) (end 24.63 0.5) (width 1) (layer "F.Cu") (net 2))
 (segment (start 34.29 52.07) (end 32.798567 53.561433) (width 1) (layer "F.Cu") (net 13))
 (segment (start 22.86 33.02) (end 34.29 44.45) (width 1) (layer "F.Cu") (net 13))
 (segment (start 11.43 31.75) (end 12.7 33.02) (width 1) (layer "F.Cu") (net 13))
 (segment (start 12.7 33.02) (end 22.86 33.02) (width 1) (layer "F.Cu") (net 13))
 (segment (start 11.43 27.94) (end 11.43 31.75) (width 1) (layer "F.Cu") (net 13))
 (segment (start 34.29 44.45) (end 34.29 52.07) (width 1) (layer "F.Cu") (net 13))
 (segment (start 6.35 25.4) (end 8.89 25.4) (width 1) (layer "F.Cu") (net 13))
 (segment (start 8.89 25.4) (end 11.43 27.94) (width 1) (layer "F.Cu") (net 13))
 (segment (start 32.798567 53.561433) (end 32.798567 78.996788) (width 1) (layer "F.Cu") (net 13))
 (segment (start 29.21 79.000323) (end 29.21 53.34) (width 1) (layer "F.Cu") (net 14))
 (segment (start 8.89 34.29) (end 10.16 35.56) (width 1) (layer "F.Cu") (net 14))
 (segment (start 31.75 45.72) (end 21.59 35.56) (width 1) (layer "F.Cu") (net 14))
 (segment (start 8.89 29.21) (end 8.89 34.29) (width 1) (layer "F.Cu") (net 14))
 (segment (start 31.002516 80.792839) (end 29.21 79.000323) (width 1) (layer "F.Cu") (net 14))
 (segment (start 31.75 50.8) (end 31.75 45.72) (width 1) (layer "F.Cu") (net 14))
 (segment (start 6.35 27.94) (end 7.62 27.94) (width 1) (layer "F.Cu") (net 14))
 (segment (start 29.21 53.34) (end 31.75 50.8) (width 1) (layer "F.Cu") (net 14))
 (segment (start 10.16 35.56) (end 21.59 35.56) (width 1) (layer "F.Cu") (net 14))
 (segment (start 7.62 27.94) (end 8.89 29.21) (width 1) (layer "F.Cu") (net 14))
 (segment (start 20.32 38.1) (end 29.21 46.99) (width 1) (layer "F.Cu") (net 15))
 (segment (start 29.21 49.53) (end 26.67 52.07) (width 1) (layer "F.Cu") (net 15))
 (segment (start 26.67 52.07) (end 26.67 80.052425) (width 1) (layer "F.Cu") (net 15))
 (segment (start 6.35 36.83) (end 7.62 38.1) (width 1) (layer "F.Cu") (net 15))
 (segment (start 29.21 46.99) (end 29.21 49.53) (width 1) (layer "F.Cu") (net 15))
 (segment (start 6.35 30.48) (end 6.35 36.83) (width 1) (layer "F.Cu") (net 15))
 (segment (start 26.67 80.052425) (end 29.206465 82.58889) (width 1) (layer "F.Cu") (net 15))
 (segment (start 7.62 38.1) (end 20.32 38.1) (width 1) (layer "F.Cu") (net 15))
 (segment (start 24.13 30.48) (end 36.83 43.18) (width 1) (layer "F.Cu") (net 8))
 (segment (start 21.59 30.48) (end 24.13 30.48) (width 1) (layer "F.Cu") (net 8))
 (segment (start 30.48 86.36) (end 29.385471 86.36) (width 1) (layer "F.Cu") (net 8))
 (segment (start 36.83 80.01) (end 30.48 86.36) (width 1) (layer "F.Cu") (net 8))
 (segment (start 36.83 43.18) (end 36.83 80.01) (width 1) (layer "F.Cu") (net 8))
 (segment (start 29.385471 86.36) (end 27.410413 84.384942) (width 1) (layer "F.Cu") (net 8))
 (segment (start -27.785922 7.991973) (end -25.617895 10.16) (width 1) (layer "F.Cu") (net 19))
 (segment (start -21.59 11.43) (end -21.59 15.24) (width 1) (layer "F.Cu") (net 19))
 (segment (start -22.86 10.16) (end -21.59 11.43) (width 1) (layer "F.Cu") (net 19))
 (segment (start -25.617895 10.16) (end -22.86 10.16) (width 1) (layer "F.Cu") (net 19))
 (segment (start -22.86 17.78) (end -21.59 17.78) (width 1) (layer "F.Cu") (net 18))
 (segment (start -25.4 15.24) (end -22.86 17.78) (width 1) (layer "F.Cu") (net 18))
 (segment (start -25.4 13.97) (end -25.4 15.24) (width 1) (layer "F.Cu") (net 18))
 (segment (start -29.581974 9.788025) (end -25.4 13.97) (width 1) (layer "F.Cu") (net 18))
 (segment (start -27.94 15.022101) (end -27.94 17.78) (width 1) (layer "F.Cu") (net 17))
 (segment (start -27.94 17.78) (end -25.4 20.32) (width 1) (layer "F.Cu") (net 17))
 (segment (start -25.4 20.32) (end -21.59 20.32) (width 1) (layer "F.Cu") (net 17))
 (segment (start -31.378025 11.584076) (end -27.94 15.022101) (width 1) (layer "F.Cu") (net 17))
 (segment (start -26.67 22.86) (end -21.59 22.86) (width 1) (layer "F.Cu") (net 16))
 (segment (start -33.174076 13.380127) (end -33.174076 16.355924) (width 1) (layer "F.Cu") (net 16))
 (segment (start -33.174076 16.355924) (end -26.67 22.86) (width 1) (layer "F.Cu") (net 16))
 (segment (start -1.24 29.24) (end -1.24 38.16) (width 1) (layer "F.Cu") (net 1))
 (segment (start 1.27 8.89) (end 2.54 10.16) (width 1) (layer "F.Cu") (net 1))
 (segment (start 2.54 10.16) (end 2.54 25.4) (width 1) (layer "F.Cu") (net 1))
 (segment (start -1.27 29.21) (end -1.24 29.24) (width 1) (layer "F.Cu") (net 1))
 (segment (start 2.54 25.4) (end -1.27 29.21) (width 1) (layer "F.Cu") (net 1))
 (segment (start 0 8.89) (end 1.27 8.89) (width 1) (layer "F.Cu") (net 1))
 (segment (start 17.145 3.175) (end -1.905 3.175) (width 1) (layer "F.Cu") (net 20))
 (segment (start -3.81 15.24) (end 0 11.43) (width 1) (layer "F.Cu") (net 20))
 (segment (start -6.35 15.24) (end -3.81 15.24) (width 1) (layer "F.Cu") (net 20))
 (segment (start -2.54 11.43) (end -3.81 10.16) (width 1) (layer "F.Cu") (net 20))
 (segment (start -1.905 3.175) (end -3.81 5.08) (width 1) (layer "F.Cu") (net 20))
 (segment (start 0 11.43) (end -2.54 11.43) (width 1) (layer "F.Cu") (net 20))
 (segment (start -3.81 10.16) (end -3.81 5.08) (width 1) (layer "F.Cu") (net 20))
 (segment (start -30.48 27.94) (end -30.48 80.227895) (width 1) (layer "F.Cu") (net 27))
 (segment (start -21.59 25.4) (end -27.94 25.4) (width 1) (layer "F.Cu") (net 27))
 (segment (start -30.48 80.227895) (end -31.378027 81.125922) (width 1) (layer "F.Cu") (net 27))
 (segment (start -27.94 25.4) (end -30.48 27.94) (width 1) (layer "F.Cu") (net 27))
 (segment (start -27.94 81.279999) (end -27.94 29.21) (width 1) (layer "F.Cu") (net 28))
 (segment (start -27.94 29.21) (end -26.67 27.94) (width 1) (layer "F.Cu") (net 28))
 (segment (start -29.581975 82.921974) (end -27.94 81.279999) (width 1) (layer "F.Cu") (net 28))
 (segment (start -26.67 27.94) (end -21.59 27.94) (width 1) (layer "F.Cu") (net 28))
 (segment (start -25.4 31.75) (end -25.4 82.332101) (width 1) (layer "F.Cu") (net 29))
 (segment (start -21.59 30.48) (end -24.13 30.48) (width 1) (layer "F.Cu") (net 29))
 (segment (start -24.13 30.48) (end -25.4 31.75) (width 1) (layer "F.Cu") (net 29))
 (segment (start -25.4 82.332101) (end -27.785924 84.718025) (width 1) (layer "F.Cu") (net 29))
 (segment (start -7.62 33.02) (end -6.35 31.75) (width 1) (layer "F.Cu") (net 26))
 (segment (start -22.86 34.29) (end -21.59 33.02) (width 1) (layer "F.Cu") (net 26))
 (segment (start -25.989873 86.514076) (end -22.86 83.384203) (width 1) (layer "F.Cu") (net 26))
 (segment (start -6.35 31.75) (end -6.35 30.48) (width 1) (layer "F.Cu") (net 26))
 (segment (start -22.86 83.384203) (end -22.86 34.29) (width 1) (layer "F.Cu") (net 26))
 (segment (start -21.59 33.02) (end -7.62 33.02) (width 1) (layer "F.Cu") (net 26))
 (segment (start 17.145 16.51) (end 18.415 15.24) (width 1) (layer "F.Cu") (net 3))
 (segment (start 18.415 15.24) (end 21.59 15.24) (width 1) (layer "F.Cu") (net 3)))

